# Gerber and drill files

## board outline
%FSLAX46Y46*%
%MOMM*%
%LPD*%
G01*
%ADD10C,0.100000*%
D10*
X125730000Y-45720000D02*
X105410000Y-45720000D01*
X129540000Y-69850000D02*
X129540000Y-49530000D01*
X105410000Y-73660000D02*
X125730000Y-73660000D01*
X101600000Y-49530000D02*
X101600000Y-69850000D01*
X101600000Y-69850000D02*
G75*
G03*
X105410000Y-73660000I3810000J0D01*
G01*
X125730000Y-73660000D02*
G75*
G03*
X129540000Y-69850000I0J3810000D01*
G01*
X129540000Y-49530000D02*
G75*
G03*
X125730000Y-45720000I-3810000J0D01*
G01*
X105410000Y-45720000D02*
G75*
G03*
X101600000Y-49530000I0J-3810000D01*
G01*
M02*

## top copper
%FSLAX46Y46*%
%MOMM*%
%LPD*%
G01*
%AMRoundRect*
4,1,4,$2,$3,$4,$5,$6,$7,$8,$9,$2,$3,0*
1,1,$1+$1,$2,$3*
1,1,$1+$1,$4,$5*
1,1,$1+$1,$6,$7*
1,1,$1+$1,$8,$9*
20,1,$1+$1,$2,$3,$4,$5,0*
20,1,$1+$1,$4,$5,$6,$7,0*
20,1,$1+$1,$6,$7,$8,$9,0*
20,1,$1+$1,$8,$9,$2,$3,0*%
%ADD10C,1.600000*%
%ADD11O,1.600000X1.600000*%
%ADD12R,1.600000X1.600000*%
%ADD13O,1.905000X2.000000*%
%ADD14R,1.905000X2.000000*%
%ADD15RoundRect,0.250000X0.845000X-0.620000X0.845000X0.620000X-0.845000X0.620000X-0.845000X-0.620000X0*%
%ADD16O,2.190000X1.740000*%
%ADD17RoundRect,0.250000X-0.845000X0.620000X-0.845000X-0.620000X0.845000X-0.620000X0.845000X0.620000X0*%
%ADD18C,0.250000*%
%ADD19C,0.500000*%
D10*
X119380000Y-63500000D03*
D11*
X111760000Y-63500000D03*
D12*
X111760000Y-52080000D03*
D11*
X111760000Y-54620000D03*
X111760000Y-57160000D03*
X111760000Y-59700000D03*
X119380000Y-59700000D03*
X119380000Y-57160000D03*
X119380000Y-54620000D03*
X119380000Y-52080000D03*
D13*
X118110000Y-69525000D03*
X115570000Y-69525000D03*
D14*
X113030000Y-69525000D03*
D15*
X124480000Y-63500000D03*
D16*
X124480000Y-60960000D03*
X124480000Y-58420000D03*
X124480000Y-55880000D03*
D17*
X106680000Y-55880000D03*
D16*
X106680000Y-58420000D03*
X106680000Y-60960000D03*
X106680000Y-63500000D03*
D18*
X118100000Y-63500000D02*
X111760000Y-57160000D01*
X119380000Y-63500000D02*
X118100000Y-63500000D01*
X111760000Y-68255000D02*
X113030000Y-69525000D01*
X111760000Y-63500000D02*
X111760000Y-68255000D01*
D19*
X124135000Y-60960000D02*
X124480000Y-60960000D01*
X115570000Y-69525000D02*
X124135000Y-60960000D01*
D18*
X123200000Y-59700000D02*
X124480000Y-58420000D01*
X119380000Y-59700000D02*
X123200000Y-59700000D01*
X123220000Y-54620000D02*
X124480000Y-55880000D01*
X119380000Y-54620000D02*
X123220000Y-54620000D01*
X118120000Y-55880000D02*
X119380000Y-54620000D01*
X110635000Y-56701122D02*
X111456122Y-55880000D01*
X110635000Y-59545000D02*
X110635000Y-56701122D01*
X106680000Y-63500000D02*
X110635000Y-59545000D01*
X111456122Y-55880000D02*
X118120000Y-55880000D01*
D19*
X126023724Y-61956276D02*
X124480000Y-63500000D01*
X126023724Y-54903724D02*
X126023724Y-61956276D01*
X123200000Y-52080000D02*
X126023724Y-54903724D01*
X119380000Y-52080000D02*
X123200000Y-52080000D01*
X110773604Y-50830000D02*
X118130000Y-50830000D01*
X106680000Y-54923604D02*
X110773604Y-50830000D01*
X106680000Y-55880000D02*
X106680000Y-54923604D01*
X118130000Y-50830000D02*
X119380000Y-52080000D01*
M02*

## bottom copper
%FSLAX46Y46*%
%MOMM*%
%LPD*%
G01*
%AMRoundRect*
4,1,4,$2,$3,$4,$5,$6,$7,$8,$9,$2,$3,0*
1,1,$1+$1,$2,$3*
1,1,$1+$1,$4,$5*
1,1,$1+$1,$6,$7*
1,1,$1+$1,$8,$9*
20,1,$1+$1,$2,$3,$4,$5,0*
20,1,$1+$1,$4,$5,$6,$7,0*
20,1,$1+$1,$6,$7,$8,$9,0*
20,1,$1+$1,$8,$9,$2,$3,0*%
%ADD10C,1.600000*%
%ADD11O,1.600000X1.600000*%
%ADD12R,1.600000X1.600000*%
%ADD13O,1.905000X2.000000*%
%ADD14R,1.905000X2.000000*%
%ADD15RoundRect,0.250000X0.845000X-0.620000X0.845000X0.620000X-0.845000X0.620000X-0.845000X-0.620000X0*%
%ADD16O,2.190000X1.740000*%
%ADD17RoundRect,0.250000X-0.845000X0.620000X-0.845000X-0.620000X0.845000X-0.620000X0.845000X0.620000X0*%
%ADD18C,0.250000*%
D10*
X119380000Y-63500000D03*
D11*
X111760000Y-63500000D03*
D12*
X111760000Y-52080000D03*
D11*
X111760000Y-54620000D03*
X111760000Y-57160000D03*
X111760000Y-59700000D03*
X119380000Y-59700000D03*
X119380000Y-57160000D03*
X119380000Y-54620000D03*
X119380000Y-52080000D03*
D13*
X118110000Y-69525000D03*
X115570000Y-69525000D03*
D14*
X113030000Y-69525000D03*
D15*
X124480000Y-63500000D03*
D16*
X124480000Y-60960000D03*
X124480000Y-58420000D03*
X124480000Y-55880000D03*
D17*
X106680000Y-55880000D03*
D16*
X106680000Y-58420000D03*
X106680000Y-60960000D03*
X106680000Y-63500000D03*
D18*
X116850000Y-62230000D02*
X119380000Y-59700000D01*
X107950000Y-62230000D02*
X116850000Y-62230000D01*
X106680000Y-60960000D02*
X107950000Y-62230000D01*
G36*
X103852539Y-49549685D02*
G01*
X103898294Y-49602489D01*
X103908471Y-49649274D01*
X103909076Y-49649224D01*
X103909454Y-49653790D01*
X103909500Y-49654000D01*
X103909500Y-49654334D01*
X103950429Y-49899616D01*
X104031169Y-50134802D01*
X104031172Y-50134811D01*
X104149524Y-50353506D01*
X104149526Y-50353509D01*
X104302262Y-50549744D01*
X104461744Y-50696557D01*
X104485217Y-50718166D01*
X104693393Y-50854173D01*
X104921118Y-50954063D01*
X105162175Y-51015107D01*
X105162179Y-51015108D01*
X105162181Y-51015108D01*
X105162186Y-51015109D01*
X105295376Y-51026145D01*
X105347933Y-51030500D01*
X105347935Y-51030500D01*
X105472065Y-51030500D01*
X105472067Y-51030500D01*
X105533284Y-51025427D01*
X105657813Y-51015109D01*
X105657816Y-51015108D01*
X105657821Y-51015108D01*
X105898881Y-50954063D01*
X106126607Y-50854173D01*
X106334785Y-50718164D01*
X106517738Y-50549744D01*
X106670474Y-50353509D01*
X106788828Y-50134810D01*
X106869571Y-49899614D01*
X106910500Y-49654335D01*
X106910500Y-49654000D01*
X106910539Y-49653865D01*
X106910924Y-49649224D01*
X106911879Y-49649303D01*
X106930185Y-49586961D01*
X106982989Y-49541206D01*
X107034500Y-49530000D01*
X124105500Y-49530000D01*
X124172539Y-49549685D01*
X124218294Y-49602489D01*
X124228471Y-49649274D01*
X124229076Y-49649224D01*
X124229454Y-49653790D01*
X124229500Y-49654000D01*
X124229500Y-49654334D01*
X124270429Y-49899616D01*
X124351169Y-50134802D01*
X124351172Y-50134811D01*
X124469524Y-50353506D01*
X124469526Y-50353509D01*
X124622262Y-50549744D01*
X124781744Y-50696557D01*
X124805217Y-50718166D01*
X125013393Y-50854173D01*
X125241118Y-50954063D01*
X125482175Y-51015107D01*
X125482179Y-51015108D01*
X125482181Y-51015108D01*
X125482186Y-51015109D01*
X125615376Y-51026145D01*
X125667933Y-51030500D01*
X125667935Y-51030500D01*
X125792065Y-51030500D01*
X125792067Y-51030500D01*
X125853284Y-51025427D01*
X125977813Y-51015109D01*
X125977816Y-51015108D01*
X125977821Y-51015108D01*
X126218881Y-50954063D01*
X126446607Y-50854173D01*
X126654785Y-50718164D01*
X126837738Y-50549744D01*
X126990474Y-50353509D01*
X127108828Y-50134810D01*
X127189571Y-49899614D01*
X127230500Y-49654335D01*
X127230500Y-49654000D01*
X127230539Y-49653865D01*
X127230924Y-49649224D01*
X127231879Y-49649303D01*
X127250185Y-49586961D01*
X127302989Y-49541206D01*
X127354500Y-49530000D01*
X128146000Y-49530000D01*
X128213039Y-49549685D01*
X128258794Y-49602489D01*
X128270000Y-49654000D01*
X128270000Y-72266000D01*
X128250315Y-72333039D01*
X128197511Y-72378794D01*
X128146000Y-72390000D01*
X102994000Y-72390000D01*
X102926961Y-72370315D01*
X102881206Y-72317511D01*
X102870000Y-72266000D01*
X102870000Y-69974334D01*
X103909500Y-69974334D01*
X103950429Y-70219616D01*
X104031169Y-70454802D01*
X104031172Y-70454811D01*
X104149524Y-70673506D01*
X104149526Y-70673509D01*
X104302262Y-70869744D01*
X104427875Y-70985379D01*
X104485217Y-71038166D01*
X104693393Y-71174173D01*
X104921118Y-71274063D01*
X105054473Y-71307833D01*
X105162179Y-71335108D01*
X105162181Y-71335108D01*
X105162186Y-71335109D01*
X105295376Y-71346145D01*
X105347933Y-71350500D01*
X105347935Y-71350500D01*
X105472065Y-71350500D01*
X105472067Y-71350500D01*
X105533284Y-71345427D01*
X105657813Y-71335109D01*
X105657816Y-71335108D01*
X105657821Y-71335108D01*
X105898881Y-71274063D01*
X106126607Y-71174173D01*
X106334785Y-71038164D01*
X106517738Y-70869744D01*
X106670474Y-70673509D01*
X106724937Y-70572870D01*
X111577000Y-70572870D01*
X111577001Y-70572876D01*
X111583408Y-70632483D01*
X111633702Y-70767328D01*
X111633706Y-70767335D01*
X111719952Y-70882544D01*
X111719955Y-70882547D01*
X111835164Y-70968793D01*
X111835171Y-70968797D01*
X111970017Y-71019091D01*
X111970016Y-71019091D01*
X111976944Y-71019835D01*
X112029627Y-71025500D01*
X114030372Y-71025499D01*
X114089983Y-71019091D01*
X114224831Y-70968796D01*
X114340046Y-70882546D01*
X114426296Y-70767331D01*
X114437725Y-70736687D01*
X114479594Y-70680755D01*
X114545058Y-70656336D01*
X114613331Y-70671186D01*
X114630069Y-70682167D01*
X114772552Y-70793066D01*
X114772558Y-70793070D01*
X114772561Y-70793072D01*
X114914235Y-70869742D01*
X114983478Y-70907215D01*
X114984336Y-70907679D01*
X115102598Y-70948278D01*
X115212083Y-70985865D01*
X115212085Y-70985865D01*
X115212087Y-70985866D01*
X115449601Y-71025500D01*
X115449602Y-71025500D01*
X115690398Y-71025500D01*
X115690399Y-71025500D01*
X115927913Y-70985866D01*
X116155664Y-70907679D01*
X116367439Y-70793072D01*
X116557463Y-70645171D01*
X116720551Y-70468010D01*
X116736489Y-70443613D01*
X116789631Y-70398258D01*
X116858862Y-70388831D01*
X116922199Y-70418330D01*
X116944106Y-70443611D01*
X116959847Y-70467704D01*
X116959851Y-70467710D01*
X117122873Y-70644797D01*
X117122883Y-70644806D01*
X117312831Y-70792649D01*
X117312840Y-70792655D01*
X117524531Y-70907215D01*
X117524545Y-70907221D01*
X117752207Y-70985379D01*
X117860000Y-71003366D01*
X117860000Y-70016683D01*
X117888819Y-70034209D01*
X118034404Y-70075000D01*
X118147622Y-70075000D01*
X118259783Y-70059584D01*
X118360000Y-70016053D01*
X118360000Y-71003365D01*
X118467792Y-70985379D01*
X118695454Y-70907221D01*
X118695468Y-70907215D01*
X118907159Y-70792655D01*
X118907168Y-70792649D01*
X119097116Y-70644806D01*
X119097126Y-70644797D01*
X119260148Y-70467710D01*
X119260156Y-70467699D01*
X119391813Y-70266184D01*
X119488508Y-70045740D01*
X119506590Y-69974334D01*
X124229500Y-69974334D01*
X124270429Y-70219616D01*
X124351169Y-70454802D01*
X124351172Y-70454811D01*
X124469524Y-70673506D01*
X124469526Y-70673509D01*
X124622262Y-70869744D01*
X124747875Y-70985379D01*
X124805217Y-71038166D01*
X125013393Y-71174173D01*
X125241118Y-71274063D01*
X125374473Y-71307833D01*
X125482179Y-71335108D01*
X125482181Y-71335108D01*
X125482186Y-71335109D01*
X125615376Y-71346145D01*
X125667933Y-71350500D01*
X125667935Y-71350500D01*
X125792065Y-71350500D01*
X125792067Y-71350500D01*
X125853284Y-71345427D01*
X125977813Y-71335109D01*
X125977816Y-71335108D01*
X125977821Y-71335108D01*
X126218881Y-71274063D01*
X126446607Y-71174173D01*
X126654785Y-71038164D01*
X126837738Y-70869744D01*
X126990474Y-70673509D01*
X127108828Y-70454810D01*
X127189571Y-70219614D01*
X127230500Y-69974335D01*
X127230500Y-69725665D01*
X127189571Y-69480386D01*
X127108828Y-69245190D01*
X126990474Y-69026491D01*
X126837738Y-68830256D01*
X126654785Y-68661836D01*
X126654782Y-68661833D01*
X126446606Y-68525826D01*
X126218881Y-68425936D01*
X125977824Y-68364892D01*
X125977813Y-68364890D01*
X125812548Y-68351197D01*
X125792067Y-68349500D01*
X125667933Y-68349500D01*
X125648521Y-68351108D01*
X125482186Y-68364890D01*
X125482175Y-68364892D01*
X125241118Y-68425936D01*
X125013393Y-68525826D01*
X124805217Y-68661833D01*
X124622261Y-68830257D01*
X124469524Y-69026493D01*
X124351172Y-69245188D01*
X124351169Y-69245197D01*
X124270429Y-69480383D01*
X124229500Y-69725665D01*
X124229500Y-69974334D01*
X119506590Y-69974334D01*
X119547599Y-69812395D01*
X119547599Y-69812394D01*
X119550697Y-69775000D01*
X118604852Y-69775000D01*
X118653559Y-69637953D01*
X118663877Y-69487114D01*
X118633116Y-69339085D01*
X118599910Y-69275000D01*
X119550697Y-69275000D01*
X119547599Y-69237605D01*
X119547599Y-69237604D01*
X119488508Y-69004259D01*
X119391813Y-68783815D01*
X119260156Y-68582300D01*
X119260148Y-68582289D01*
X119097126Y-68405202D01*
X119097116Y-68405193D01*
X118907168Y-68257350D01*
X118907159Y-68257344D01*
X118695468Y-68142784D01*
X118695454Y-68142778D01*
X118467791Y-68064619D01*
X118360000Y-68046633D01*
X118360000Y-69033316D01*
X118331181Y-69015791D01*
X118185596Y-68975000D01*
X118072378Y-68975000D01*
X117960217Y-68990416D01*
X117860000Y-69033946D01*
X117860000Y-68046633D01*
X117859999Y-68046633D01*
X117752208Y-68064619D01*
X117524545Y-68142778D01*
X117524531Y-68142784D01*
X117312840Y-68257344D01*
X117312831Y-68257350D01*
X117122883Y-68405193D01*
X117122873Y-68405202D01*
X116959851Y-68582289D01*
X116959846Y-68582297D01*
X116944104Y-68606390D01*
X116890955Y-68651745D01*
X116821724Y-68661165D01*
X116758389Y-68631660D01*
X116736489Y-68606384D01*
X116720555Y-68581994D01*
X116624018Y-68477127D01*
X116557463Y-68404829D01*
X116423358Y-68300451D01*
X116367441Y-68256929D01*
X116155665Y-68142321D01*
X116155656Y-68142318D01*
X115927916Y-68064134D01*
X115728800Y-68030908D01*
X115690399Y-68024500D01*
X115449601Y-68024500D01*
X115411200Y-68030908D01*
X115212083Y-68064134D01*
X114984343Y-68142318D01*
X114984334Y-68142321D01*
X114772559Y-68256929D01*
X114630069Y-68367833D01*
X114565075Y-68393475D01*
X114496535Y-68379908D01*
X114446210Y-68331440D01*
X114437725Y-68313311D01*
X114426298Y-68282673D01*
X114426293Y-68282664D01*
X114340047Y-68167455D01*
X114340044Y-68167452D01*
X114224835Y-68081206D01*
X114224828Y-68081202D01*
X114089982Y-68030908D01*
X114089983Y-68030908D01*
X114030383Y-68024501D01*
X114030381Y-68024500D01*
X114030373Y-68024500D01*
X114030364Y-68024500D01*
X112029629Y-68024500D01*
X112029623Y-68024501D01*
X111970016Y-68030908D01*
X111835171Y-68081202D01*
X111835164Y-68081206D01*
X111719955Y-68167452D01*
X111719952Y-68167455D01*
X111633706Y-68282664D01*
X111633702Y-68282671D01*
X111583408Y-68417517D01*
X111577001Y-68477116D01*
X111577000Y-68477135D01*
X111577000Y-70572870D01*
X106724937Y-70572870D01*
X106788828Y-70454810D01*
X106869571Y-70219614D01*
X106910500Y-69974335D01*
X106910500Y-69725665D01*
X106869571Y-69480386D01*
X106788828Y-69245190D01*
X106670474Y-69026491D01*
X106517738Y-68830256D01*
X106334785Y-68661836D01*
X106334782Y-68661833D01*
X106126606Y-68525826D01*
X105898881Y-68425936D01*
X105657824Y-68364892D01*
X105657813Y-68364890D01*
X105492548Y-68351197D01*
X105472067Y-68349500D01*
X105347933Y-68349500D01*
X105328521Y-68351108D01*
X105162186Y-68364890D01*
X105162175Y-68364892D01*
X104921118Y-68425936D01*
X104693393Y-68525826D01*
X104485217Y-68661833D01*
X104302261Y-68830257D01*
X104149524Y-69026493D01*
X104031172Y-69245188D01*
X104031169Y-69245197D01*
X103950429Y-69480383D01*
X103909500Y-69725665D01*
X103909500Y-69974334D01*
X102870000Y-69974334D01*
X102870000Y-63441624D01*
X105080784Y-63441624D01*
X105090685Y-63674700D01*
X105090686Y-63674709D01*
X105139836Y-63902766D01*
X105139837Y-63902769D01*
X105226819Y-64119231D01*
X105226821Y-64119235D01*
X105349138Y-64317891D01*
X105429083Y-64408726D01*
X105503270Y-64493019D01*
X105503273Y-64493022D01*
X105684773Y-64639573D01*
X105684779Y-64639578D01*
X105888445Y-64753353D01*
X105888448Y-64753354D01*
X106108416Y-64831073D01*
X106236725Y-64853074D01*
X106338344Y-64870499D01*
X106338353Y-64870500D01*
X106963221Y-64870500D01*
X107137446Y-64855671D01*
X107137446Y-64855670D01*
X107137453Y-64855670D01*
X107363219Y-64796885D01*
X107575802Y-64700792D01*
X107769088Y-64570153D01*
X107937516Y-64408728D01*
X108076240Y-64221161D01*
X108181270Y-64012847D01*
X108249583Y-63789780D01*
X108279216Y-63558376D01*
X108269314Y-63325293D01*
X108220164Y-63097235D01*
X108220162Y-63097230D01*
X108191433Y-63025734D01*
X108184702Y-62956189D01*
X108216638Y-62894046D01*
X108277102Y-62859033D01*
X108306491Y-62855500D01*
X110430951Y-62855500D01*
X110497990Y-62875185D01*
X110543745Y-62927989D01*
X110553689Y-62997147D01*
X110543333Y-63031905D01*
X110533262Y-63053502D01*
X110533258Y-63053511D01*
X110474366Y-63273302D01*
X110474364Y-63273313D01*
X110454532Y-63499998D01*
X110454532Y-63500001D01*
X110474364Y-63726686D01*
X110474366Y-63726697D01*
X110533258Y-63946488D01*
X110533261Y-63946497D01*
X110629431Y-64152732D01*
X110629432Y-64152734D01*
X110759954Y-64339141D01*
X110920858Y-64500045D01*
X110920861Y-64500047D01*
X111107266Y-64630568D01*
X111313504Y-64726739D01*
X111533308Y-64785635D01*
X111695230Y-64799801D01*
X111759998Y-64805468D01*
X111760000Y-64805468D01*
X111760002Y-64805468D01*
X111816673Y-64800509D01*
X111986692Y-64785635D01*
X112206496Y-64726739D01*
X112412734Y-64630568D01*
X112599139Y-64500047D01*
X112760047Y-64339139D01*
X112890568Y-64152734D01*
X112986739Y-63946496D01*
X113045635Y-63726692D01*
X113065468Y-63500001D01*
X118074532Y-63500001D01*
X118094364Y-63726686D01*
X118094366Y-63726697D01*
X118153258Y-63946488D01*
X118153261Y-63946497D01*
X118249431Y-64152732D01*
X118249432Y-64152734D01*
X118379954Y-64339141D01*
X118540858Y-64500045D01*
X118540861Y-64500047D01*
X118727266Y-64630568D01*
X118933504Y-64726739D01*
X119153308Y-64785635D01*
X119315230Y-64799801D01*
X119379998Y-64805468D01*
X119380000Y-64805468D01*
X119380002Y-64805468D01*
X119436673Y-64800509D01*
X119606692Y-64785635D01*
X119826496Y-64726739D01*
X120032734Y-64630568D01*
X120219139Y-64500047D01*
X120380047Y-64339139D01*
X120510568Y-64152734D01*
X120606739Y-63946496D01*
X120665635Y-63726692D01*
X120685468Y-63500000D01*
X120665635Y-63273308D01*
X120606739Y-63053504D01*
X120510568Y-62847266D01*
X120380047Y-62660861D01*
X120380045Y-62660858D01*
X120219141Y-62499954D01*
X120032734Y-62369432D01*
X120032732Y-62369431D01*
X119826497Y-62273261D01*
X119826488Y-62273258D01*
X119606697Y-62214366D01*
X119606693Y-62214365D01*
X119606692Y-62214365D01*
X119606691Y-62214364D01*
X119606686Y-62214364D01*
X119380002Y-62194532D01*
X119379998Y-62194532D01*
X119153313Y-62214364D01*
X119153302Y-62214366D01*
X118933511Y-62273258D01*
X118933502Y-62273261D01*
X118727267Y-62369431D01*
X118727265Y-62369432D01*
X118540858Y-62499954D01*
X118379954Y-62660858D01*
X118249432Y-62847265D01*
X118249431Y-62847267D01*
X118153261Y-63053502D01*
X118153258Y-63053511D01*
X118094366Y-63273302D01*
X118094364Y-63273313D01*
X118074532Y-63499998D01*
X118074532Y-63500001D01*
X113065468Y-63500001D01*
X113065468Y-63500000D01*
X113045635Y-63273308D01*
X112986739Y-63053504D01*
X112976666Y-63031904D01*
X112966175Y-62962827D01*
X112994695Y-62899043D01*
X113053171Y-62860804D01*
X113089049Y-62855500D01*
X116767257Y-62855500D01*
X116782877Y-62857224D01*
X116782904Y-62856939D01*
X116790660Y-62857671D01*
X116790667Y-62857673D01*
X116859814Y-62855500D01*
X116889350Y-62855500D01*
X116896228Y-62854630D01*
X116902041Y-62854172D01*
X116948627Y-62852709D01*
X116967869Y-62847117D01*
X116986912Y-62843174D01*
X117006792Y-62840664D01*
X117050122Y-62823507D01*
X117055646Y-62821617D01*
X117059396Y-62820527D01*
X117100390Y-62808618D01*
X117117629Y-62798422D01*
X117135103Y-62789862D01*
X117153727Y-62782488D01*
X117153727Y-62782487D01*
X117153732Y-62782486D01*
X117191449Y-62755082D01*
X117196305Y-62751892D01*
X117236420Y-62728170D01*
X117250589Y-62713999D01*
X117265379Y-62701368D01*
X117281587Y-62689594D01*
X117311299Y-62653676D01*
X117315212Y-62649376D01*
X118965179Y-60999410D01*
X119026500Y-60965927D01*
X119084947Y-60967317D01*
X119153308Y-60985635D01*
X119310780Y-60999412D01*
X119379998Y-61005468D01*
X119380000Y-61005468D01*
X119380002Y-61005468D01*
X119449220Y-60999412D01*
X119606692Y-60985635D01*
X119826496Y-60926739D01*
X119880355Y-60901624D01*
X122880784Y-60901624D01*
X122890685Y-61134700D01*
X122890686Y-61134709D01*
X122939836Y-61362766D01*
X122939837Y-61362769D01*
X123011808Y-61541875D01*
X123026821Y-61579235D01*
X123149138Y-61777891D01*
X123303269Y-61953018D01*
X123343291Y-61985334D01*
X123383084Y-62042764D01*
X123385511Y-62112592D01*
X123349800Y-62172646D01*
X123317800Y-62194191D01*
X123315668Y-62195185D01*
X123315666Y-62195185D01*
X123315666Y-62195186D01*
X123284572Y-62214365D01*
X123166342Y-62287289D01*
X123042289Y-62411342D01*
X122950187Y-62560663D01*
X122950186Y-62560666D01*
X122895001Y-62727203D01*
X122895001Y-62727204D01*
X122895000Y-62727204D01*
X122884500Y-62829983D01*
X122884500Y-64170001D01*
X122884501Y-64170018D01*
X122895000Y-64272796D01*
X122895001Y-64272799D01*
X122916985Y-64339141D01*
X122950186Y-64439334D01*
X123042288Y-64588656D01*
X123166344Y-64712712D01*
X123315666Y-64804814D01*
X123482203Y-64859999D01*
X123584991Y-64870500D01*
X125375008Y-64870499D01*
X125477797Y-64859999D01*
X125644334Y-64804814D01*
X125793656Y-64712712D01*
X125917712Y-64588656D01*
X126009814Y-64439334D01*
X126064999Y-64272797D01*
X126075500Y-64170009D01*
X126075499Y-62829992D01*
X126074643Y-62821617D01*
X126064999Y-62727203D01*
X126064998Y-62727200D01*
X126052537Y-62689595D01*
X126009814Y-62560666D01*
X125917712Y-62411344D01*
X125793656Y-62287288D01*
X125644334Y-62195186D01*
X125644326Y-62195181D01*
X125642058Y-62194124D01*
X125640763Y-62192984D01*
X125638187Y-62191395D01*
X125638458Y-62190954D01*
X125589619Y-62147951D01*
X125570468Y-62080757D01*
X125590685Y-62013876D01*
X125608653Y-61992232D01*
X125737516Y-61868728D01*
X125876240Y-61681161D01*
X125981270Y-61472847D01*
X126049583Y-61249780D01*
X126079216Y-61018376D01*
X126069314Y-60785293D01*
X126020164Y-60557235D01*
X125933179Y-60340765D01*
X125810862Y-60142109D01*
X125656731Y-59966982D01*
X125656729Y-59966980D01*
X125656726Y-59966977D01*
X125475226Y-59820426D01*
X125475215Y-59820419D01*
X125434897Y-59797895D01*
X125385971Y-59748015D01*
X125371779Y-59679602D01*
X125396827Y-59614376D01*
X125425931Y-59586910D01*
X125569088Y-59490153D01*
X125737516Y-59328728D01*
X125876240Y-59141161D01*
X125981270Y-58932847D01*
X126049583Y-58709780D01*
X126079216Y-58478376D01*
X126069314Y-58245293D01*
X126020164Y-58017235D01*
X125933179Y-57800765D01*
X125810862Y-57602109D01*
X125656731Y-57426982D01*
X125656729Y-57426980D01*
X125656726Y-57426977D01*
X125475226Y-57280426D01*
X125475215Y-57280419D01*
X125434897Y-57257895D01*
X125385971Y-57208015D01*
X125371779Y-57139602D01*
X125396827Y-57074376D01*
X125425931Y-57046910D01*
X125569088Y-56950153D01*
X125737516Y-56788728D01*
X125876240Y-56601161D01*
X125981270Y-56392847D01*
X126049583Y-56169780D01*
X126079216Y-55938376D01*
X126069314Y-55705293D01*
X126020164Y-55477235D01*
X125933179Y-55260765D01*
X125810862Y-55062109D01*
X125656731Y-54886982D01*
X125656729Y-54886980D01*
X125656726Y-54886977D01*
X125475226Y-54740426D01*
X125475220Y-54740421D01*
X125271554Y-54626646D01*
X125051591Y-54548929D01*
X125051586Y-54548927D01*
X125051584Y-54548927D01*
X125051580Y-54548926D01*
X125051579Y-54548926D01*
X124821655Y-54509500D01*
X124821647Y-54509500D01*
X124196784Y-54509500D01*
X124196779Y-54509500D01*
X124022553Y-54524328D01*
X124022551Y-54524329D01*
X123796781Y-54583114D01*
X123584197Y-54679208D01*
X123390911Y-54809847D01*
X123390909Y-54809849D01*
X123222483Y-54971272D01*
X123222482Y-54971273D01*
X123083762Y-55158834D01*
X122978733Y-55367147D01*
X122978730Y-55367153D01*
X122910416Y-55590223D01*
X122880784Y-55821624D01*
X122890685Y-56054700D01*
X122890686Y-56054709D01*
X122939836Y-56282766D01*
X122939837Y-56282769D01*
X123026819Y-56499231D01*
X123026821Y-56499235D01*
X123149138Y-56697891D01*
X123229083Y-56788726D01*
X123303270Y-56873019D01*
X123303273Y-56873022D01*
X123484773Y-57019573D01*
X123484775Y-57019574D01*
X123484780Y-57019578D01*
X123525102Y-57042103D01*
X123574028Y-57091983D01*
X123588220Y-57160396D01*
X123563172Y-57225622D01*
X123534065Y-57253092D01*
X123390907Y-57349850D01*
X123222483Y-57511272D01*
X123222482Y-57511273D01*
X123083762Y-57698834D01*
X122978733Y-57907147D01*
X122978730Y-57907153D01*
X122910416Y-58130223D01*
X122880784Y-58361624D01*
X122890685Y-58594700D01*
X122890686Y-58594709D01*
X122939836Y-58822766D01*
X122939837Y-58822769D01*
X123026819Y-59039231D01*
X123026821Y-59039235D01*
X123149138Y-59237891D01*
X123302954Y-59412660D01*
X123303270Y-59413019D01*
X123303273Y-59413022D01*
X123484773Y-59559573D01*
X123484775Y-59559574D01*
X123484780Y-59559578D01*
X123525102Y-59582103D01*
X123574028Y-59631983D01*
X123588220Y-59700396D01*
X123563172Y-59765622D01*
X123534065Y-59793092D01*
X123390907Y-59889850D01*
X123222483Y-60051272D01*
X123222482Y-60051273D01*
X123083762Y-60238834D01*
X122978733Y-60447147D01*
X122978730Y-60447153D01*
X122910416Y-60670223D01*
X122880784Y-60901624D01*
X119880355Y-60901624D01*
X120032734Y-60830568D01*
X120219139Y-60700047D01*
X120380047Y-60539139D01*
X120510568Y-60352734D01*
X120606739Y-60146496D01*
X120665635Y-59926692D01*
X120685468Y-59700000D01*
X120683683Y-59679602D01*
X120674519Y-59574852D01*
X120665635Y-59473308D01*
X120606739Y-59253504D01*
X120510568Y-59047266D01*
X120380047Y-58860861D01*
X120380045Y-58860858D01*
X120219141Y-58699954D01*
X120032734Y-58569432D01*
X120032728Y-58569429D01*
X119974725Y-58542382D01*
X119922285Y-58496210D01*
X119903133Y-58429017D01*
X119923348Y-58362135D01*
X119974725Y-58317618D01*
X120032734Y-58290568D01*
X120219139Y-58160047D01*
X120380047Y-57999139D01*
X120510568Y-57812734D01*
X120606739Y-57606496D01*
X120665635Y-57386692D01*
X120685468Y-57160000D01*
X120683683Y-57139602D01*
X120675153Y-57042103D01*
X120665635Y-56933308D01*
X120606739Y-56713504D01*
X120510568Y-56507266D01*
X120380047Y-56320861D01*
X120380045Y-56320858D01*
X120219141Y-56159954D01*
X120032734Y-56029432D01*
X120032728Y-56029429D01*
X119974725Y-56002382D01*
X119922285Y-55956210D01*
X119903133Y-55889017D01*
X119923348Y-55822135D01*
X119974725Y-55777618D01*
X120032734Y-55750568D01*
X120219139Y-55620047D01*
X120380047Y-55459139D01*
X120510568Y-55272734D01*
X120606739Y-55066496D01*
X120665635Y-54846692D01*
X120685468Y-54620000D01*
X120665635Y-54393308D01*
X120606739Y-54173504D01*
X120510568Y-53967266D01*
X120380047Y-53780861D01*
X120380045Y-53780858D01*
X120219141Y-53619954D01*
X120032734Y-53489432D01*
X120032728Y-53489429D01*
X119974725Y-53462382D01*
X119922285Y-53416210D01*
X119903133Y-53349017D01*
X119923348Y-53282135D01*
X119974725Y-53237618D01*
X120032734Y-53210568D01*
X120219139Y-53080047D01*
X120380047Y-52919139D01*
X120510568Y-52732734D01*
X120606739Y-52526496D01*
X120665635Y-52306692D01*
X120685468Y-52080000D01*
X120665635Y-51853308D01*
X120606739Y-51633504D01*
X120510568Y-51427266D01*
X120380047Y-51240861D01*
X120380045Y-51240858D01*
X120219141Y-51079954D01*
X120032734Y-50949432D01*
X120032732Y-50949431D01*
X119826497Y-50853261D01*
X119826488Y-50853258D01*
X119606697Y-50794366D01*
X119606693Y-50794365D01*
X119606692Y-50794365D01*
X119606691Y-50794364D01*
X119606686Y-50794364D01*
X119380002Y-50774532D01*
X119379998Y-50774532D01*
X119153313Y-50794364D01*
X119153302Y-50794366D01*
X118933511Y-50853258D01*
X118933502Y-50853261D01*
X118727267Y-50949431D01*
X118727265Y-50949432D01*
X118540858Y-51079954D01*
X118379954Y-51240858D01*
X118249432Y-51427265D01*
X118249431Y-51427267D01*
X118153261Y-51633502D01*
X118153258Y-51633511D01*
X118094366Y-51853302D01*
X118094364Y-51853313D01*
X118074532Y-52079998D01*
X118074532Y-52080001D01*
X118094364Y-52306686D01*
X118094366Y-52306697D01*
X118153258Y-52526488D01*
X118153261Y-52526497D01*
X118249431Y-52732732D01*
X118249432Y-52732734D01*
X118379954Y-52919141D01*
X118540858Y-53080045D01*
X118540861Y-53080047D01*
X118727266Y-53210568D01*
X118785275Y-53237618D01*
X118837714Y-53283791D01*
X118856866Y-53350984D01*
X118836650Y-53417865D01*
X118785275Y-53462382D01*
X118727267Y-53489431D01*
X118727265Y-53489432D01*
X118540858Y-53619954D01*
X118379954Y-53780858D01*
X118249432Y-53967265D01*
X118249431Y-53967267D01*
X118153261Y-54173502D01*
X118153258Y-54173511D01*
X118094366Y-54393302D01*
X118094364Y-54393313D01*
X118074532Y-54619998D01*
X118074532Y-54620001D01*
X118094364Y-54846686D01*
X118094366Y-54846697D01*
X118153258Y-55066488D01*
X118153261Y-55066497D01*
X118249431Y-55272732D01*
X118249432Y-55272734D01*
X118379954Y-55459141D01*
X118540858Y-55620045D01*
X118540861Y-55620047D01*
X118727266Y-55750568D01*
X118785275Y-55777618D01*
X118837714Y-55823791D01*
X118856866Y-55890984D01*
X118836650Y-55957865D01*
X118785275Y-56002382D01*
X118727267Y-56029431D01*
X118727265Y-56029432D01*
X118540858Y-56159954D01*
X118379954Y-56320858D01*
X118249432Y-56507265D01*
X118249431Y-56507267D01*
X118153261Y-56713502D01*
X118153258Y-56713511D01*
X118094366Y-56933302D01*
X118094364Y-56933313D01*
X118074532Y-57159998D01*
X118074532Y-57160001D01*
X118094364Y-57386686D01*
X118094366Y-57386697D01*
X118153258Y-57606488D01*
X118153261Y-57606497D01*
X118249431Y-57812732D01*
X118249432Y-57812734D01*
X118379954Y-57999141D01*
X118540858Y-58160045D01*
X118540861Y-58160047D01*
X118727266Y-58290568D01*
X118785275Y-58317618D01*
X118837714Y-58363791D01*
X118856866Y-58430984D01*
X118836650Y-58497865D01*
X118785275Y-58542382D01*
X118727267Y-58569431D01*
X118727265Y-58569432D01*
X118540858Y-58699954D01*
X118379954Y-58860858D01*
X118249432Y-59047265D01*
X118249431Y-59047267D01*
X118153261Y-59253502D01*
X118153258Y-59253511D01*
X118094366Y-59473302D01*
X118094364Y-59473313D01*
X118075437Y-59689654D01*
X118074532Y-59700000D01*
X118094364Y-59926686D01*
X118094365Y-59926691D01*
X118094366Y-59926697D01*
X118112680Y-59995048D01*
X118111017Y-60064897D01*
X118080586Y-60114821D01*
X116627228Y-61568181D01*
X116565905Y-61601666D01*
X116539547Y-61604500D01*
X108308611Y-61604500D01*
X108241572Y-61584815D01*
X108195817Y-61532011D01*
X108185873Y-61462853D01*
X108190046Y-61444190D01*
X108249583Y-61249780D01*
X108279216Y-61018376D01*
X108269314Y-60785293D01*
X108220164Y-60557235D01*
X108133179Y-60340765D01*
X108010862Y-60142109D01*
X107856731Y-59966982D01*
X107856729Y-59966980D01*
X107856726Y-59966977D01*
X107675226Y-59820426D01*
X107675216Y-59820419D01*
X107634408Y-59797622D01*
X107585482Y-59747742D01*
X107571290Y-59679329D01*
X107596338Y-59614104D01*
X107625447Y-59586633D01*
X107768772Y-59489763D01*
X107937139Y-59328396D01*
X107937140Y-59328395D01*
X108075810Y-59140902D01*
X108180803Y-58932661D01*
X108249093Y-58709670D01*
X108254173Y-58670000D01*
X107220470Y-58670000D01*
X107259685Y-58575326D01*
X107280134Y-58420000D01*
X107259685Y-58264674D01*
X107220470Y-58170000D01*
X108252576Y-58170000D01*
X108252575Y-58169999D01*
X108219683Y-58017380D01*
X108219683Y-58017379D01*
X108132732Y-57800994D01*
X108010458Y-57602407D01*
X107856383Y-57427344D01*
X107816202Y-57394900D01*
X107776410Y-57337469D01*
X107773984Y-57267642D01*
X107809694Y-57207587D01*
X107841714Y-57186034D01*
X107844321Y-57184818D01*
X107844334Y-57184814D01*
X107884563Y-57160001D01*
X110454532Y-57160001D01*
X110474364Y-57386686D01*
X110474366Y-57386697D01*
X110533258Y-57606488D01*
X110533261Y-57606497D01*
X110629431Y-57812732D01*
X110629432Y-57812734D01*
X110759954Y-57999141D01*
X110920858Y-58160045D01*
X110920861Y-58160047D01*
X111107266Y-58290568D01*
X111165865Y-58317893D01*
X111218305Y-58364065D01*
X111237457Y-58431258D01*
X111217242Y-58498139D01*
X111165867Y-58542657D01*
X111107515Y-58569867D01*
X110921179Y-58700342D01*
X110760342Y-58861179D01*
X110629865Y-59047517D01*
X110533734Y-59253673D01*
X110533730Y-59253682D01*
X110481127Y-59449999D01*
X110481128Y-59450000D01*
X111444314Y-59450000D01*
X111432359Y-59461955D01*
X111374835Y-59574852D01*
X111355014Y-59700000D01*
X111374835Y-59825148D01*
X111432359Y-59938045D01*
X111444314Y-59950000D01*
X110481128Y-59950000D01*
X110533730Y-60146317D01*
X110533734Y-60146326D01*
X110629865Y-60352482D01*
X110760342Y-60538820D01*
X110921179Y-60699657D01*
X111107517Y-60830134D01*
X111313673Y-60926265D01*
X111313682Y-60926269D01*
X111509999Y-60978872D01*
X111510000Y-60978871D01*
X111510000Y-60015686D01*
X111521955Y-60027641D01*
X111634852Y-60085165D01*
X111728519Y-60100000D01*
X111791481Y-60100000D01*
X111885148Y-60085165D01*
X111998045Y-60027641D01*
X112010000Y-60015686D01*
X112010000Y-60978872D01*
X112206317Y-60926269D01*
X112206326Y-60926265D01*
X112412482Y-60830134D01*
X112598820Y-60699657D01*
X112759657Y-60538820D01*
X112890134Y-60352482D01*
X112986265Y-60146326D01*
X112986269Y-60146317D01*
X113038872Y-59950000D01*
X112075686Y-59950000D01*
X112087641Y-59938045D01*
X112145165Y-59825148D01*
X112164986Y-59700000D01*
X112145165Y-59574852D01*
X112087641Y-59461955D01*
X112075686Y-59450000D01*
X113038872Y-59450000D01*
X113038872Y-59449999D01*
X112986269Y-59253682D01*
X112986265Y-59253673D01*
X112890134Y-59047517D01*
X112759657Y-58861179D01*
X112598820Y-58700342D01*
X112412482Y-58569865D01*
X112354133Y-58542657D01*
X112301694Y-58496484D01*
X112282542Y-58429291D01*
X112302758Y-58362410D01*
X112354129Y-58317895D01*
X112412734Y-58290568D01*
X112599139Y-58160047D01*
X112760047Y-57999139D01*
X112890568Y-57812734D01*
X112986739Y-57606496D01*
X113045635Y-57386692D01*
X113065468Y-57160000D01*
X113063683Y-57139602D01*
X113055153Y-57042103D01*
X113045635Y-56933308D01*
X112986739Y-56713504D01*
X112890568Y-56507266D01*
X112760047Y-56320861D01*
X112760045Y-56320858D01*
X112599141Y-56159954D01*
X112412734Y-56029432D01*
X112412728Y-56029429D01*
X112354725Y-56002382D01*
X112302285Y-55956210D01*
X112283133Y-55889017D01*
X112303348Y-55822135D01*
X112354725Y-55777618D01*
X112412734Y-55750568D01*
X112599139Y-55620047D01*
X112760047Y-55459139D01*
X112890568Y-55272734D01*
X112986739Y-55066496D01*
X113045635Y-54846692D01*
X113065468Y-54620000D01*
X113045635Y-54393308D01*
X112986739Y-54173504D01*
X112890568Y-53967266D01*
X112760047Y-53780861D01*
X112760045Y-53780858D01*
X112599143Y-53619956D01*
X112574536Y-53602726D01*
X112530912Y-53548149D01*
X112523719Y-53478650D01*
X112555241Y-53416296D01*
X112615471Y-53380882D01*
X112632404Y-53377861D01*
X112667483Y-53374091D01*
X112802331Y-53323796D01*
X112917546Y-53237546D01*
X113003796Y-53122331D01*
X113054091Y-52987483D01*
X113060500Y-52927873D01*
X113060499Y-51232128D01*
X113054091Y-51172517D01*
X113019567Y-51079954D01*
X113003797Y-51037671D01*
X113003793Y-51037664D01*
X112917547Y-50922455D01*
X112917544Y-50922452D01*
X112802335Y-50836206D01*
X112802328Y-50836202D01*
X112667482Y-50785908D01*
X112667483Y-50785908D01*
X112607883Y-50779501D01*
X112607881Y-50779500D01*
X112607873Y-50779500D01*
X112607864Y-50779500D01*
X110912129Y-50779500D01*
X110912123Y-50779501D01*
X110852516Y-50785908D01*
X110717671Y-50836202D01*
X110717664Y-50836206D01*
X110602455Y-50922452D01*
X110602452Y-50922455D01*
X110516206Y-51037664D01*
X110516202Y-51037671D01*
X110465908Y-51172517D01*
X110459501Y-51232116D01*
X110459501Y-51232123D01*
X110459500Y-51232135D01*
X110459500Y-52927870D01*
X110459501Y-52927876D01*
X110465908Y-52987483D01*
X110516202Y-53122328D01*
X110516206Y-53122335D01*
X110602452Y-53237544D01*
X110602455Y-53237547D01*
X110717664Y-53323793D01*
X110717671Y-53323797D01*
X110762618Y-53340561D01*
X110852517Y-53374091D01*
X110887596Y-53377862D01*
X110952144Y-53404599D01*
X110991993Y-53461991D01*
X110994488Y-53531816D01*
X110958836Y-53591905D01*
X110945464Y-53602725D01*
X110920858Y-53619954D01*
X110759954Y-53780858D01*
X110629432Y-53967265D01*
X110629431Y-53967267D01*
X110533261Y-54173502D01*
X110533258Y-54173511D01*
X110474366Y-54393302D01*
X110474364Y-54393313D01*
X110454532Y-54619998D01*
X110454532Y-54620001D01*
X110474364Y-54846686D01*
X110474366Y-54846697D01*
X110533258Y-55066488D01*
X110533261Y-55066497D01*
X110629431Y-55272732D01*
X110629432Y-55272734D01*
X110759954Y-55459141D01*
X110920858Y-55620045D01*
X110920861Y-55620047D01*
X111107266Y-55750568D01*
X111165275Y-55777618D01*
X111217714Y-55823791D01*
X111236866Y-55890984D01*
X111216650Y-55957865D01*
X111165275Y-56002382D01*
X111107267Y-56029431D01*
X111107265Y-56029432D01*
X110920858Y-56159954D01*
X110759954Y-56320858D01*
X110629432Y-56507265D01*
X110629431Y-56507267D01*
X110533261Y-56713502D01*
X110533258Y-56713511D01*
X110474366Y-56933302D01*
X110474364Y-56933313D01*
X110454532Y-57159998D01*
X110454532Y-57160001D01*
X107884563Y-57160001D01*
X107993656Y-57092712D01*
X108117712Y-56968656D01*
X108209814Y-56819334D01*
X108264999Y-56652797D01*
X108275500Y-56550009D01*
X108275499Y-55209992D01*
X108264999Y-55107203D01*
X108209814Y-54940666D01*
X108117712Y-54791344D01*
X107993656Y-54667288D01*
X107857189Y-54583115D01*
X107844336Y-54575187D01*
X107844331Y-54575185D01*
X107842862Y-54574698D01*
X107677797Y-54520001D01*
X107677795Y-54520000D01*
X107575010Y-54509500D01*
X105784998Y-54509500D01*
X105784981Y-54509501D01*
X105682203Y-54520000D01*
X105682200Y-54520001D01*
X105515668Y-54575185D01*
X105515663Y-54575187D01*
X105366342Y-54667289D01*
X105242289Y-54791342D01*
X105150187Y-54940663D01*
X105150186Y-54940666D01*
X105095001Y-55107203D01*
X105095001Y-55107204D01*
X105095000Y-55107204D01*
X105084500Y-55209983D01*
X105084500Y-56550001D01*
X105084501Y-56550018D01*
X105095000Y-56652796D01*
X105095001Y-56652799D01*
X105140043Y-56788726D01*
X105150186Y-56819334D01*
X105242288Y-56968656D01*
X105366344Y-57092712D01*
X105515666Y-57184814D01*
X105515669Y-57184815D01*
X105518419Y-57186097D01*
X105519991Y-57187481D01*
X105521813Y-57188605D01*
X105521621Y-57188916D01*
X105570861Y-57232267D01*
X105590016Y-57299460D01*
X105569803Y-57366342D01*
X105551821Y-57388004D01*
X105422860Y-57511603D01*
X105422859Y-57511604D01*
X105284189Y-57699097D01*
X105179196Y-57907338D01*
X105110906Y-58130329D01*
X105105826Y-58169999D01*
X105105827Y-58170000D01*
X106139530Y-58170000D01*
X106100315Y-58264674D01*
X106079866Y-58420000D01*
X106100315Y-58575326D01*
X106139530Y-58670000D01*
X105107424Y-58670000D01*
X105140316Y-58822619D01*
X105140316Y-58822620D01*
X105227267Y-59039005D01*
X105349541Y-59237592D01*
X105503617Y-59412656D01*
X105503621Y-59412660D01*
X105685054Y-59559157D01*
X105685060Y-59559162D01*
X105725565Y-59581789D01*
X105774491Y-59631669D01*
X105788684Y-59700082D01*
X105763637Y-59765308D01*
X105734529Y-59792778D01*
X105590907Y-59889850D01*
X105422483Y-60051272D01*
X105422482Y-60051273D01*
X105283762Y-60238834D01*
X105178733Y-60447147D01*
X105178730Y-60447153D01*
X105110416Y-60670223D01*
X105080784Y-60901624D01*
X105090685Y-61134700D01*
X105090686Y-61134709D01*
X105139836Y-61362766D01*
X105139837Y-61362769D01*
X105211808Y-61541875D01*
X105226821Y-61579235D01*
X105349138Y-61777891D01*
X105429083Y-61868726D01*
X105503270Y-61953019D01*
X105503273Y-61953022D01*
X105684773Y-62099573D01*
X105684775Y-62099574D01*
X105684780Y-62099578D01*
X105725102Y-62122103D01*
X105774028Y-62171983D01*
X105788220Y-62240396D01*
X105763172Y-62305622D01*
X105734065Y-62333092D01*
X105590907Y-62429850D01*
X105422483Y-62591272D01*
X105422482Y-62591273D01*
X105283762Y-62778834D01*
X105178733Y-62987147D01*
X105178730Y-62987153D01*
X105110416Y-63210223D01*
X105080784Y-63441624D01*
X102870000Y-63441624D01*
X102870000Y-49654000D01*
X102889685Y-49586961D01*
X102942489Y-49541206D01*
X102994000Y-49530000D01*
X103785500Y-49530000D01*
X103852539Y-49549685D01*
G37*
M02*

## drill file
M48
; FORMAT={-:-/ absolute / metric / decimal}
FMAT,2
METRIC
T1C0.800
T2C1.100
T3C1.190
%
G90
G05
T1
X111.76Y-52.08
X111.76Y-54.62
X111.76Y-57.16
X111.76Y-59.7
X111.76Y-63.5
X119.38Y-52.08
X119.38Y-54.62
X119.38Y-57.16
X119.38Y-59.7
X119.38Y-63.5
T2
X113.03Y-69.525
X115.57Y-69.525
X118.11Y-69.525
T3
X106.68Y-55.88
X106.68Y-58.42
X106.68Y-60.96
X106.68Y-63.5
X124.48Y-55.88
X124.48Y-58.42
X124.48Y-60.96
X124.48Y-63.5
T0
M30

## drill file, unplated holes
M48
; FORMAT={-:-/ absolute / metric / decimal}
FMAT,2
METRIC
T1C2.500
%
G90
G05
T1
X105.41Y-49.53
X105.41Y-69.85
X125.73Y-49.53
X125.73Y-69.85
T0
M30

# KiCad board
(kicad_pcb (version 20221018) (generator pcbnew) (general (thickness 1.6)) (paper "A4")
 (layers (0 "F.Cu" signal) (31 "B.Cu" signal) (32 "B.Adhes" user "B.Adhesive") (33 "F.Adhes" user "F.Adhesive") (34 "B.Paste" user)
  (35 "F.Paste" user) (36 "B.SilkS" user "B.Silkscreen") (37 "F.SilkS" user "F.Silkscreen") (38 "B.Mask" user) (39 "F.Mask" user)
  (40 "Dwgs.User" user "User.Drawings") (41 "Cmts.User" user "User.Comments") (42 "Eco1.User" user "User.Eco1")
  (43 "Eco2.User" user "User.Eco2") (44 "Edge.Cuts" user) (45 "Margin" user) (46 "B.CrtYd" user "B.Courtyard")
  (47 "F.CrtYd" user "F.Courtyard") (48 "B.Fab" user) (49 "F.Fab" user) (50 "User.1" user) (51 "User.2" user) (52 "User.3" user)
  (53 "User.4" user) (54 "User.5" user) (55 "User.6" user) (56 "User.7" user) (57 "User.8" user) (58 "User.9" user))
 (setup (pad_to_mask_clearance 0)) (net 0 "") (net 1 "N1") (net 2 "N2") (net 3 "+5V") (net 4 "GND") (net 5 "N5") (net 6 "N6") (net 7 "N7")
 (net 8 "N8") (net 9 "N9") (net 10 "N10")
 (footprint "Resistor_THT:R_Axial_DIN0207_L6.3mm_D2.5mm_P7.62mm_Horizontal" (layer "F.Cu") (at 119.38 63.5 180)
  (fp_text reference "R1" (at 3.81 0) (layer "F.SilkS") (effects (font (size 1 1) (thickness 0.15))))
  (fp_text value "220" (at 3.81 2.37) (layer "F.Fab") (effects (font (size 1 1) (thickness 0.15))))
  (pad "1" thru_hole circle (at 0 0 180) (size 1.6 1.6) (drill 0.8) (layers "*.Cu" "*.Mask") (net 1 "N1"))
  (pad "2" thru_hole oval (at 7.62 0 180) (size 1.6 1.6) (drill 0.8) (layers "*.Cu" "*.Mask") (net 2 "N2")))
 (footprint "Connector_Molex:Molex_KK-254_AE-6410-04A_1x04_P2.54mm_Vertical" (layer "F.Cu") (at 106.68 55.88 -90)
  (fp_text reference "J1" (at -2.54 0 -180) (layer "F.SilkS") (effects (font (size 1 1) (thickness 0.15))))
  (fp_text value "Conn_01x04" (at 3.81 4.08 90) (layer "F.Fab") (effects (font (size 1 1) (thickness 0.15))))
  (pad "1" thru_hole roundrect (at 0 0 270) (size 1.74 2.19) (drill 1.19) (layers "*.Cu" "*.Mask") (roundrect_rratio 0.1436781609)
   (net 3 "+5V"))
  (pad "2" thru_hole oval (at 2.54 0 270) (size 1.74 2.19) (drill 1.19) (layers "*.Cu" "*.Mask") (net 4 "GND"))
  (pad "3" thru_hole oval (at 5.08 0 270) (size 1.74 2.19) (drill 1.19) (layers "*.Cu" "*.Mask") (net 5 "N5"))
  (pad "4" thru_hole oval (at 7.62 0 270) (size 1.74 2.19) (drill 1.19) (layers "*.Cu" "*.Mask") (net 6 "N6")))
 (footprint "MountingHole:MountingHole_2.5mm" (layer "F.Cu") (at 125.73 49.53)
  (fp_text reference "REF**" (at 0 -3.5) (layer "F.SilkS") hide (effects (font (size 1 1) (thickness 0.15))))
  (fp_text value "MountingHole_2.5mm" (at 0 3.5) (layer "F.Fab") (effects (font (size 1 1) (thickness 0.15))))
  (pad "" np_thru_hole circle (at 0 0) (size 2.5 2.5) (drill 2.5) (layers "*.Cu" "*.Mask")))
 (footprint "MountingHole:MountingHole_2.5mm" (layer "F.Cu") (at 125.73 69.85)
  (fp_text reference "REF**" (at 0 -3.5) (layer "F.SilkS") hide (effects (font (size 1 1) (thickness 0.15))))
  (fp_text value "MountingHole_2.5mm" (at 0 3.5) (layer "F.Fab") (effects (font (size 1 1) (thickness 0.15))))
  (pad "" np_thru_hole circle (at 0 0) (size 2.5 2.5) (drill 2.5) (layers "*.Cu" "*.Mask")))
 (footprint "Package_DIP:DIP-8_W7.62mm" (layer "F.Cu") (at 111.76 52.08)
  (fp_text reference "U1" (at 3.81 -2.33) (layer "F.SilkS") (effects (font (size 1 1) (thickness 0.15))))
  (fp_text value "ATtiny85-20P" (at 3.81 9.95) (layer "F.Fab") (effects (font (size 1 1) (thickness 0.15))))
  (pad "1" thru_hole rect (at 0 0) (size 1.6 1.6) (drill 0.8) (layers "*.Cu" "*.Mask") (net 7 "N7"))
  (pad "2" thru_hole oval (at 0 2.54) (size 1.6 1.6) (drill 0.8) (layers "*.Cu" "*.Mask") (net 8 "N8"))
  (pad "3" thru_hole oval (at 0 5.08) (size 1.6 1.6) (drill 0.8) (layers "*.Cu" "*.Mask") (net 1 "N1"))
  (pad "4" thru_hole oval (at 0 7.62) (size 1.6 1.6) (drill 0.8) (layers "*.Cu" "*.Mask") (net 4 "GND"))
  (pad "5" thru_hole oval (at 7.62 7.62) (size 1.6 1.6) (drill 0.8) (layers "*.Cu" "*.Mask") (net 5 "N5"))
  (pad "6" thru_hole oval (at 7.62 5.08) (size 1.6 1.6) (drill 0.8) (layers "*.Cu" "*.Mask") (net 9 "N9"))
  (pad "7" thru_hole oval (at 7.62 2.54) (size 1.6 1.6) (drill 0.8) (layers "*.Cu" "*.Mask") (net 6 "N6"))
  (pad "8" thru_hole oval (at 7.62 0) (size 1.6 1.6) (drill 0.8) (layers "*.Cu" "*.Mask") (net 3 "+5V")))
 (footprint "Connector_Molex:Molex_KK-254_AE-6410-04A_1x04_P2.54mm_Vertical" (layer "F.Cu") (at 124.48 63.5 90)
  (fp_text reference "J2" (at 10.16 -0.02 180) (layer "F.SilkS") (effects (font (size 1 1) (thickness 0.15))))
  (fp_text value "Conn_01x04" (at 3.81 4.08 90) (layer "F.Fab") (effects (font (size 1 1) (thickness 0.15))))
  (pad "1" thru_hole roundrect (at 0 0 90) (size 1.74 2.19) (drill 1.19) (layers "*.Cu" "*.Mask") (roundrect_rratio 0.1436781609)
   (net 3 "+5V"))
  (pad "2" thru_hole oval (at 2.54 0 90) (size 1.74 2.19) (drill 1.19) (layers "*.Cu" "*.Mask") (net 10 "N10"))
  (pad "3" thru_hole oval (at 5.08 0 90) (size 1.74 2.19) (drill 1.19) (layers "*.Cu" "*.Mask") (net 5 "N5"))
  (pad "4" thru_hole oval (at 7.62 0 90) (size 1.74 2.19) (drill 1.19) (layers "*.Cu" "*.Mask") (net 6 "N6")))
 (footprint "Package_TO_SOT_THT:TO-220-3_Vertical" (layer "F.Cu") (at 113.03 69.525)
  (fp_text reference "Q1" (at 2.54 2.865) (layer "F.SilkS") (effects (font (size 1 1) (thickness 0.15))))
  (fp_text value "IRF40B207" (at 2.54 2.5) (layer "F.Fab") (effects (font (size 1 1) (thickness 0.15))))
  (pad "1" thru_hole rect (at 0 0) (size 1.905 2) (drill 1.1) (layers "*.Cu" "*.Mask") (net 2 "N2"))
  (pad "2" thru_hole oval (at 2.54 0) (size 1.905 2) (drill 1.1) (layers "*.Cu" "*.Mask") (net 10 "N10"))
  (pad "3" thru_hole oval (at 5.08 0) (size 1.905 2) (drill 1.1) (layers "*.Cu" "*.Mask") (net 4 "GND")))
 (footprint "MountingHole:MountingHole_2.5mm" (layer "F.Cu") (at 105.41 69.85)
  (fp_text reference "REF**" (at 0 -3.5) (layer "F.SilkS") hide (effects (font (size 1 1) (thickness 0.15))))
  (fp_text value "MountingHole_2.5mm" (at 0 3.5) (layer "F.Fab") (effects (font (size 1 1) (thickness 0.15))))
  (pad "" np_thru_hole circle (at 0 0) (size 2.5 2.5) (drill 2.5) (layers "*.Cu" "*.Mask")))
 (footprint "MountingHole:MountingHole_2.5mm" (layer "F.Cu") (at 105.41 49.53)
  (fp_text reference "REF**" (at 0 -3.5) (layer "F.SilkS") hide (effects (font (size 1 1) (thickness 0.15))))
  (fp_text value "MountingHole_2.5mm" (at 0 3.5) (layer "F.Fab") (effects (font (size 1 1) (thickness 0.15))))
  (pad "" np_thru_hole circle (at 0 0) (size 2.5 2.5) (drill 2.5) (layers "*.Cu" "*.Mask")))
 (gr_arc (start 129.54 69.85) (mid 128.424077 72.544077) (end 125.73 73.66) (stroke (width 0.1) (type default)) (layer "Edge.Cuts"))
 (gr_arc (start 105.41 73.66) (mid 102.715923 72.544077) (end 101.6 69.85) (stroke (width 0.1) (type default)) (layer "Edge.Cuts"))
 (gr_line (start 125.73 45.72) (end 105.41 45.72) (stroke (width 0.1) (type default)) (layer "Edge.Cuts"))
 (gr_line (start 129.54 69.85) (end 129.54 49.53) (stroke (width 0.1) (type default)) (layer "Edge.Cuts"))
 (gr_line (start 101.6 49.53) (end 101.6 69.85) (stroke (width 0.1) (type default)) (layer "Edge.Cuts"))
 (gr_line (start 105.41 73.66) (end 125.73 73.66) (stroke (width 0.1) (type default)) (layer "Edge.Cuts"))
 (gr_arc (start 125.73 45.72) (mid 128.424077 46.835923) (end 129.54 49.53) (stroke (width 0.1) (type default)) (layer "Edge.Cuts"))
 (gr_arc (start 101.6 49.53) (mid 102.715923 46.835923) (end 105.41 45.72) (stroke (width 0.1) (type default)) (layer "Edge.Cuts"))
 (segment (start 118.13 50.83) (end 119.38 52.08) (width 0.5) (layer "F.Cu") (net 3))
 (segment (start 126.023724 61.956276) (end 124.48 63.5) (width 0.5) (layer "F.Cu") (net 3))
 (segment (start 119.38 52.08) (end 123.2 52.08) (width 0.5) (layer "F.Cu") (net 3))
 (segment (start 106.68 54.923604) (end 110.773604 50.83) (width 0.5) (layer "F.Cu") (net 3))
 (segment (start 110.773604 50.83) (end 118.13 50.83) (width 0.5) (layer "F.Cu") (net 3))
 (segment (start 123.2 52.08) (end 126.023724 54.903724) (width 0.5) (layer "F.Cu") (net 3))
 (segment (start 106.68 55.88) (end 106.68 54.923604) (width 0.5) (layer "F.Cu") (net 3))
 (segment (start 126.023724 54.903724) (end 126.023724 61.956276) (width 0.5) (layer "F.Cu") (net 3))
 (segment (start 123.2 59.7) (end 124.48 58.42) (width 0.25) (layer "F.Cu") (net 5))
 (segment (start 119.38 59.7) (end 123.2 59.7) (width 0.25) (layer "F.Cu") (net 5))
 (segment (start 116.85 62.23) (end 119.38 59.7) (width 0.25) (layer "B.Cu") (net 5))
 (segment (start 107.95 62.23) (end 116.85 62.23) (width 0.25) (layer "B.Cu") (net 5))
 (segment (start 106.68 60.96) (end 107.95 62.23) (width 0.25) (layer "B.Cu") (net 5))
 (segment (start 110.635 56.701122) (end 111.456122 55.88) (width 0.25) (layer "F.Cu") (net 6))
 (segment (start 111.456122 55.88) (end 118.12 55.88) (width 0.25) (layer "F.Cu") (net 6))
 (segment (start 110.635 59.545) (end 110.635 56.701122) (width 0.25) (layer "F.Cu") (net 6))
 (segment (start 106.68 63.5) (end 110.635 59.545) (width 0.25) (layer "F.Cu") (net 6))
 (segment (start 123.22 54.62) (end 124.48 55.88) (width 0.25) (layer "F.Cu") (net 6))
 (segment (start 119.38 54.62) (end 123.22 54.62) (width 0.25) (layer "F.Cu") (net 6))
 (segment (start 118.12 55.88) (end 119.38 54.62) (width 0.25) (layer "F.Cu") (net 6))
 (segment (start 115.57 69.525) (end 124.135 60.96) (width 0.5) (layer "F.Cu") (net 10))
 (segment (start 124.135 60.96) (end 124.48 60.96) (width 0.5) (layer "F.Cu") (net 10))
 (segment (start 111.76 68.255) (end 113.03 69.525) (width 0.25) (layer "F.Cu") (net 2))
 (segment (start 111.76 63.5) (end 111.76 68.255) (width 0.25) (layer "F.Cu") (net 2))
 (segment (start 118.1 63.5) (end 111.76 57.16) (width 0.25) (layer "F.Cu") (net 1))
 (segment (start 119.38 63.5) (end 118.1 63.5) (width 0.25) (layer "F.Cu") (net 1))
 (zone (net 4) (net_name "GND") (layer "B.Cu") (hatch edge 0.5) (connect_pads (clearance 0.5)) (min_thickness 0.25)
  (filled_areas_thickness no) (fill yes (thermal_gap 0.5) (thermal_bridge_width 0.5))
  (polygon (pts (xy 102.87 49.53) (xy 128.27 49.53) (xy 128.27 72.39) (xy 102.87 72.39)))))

